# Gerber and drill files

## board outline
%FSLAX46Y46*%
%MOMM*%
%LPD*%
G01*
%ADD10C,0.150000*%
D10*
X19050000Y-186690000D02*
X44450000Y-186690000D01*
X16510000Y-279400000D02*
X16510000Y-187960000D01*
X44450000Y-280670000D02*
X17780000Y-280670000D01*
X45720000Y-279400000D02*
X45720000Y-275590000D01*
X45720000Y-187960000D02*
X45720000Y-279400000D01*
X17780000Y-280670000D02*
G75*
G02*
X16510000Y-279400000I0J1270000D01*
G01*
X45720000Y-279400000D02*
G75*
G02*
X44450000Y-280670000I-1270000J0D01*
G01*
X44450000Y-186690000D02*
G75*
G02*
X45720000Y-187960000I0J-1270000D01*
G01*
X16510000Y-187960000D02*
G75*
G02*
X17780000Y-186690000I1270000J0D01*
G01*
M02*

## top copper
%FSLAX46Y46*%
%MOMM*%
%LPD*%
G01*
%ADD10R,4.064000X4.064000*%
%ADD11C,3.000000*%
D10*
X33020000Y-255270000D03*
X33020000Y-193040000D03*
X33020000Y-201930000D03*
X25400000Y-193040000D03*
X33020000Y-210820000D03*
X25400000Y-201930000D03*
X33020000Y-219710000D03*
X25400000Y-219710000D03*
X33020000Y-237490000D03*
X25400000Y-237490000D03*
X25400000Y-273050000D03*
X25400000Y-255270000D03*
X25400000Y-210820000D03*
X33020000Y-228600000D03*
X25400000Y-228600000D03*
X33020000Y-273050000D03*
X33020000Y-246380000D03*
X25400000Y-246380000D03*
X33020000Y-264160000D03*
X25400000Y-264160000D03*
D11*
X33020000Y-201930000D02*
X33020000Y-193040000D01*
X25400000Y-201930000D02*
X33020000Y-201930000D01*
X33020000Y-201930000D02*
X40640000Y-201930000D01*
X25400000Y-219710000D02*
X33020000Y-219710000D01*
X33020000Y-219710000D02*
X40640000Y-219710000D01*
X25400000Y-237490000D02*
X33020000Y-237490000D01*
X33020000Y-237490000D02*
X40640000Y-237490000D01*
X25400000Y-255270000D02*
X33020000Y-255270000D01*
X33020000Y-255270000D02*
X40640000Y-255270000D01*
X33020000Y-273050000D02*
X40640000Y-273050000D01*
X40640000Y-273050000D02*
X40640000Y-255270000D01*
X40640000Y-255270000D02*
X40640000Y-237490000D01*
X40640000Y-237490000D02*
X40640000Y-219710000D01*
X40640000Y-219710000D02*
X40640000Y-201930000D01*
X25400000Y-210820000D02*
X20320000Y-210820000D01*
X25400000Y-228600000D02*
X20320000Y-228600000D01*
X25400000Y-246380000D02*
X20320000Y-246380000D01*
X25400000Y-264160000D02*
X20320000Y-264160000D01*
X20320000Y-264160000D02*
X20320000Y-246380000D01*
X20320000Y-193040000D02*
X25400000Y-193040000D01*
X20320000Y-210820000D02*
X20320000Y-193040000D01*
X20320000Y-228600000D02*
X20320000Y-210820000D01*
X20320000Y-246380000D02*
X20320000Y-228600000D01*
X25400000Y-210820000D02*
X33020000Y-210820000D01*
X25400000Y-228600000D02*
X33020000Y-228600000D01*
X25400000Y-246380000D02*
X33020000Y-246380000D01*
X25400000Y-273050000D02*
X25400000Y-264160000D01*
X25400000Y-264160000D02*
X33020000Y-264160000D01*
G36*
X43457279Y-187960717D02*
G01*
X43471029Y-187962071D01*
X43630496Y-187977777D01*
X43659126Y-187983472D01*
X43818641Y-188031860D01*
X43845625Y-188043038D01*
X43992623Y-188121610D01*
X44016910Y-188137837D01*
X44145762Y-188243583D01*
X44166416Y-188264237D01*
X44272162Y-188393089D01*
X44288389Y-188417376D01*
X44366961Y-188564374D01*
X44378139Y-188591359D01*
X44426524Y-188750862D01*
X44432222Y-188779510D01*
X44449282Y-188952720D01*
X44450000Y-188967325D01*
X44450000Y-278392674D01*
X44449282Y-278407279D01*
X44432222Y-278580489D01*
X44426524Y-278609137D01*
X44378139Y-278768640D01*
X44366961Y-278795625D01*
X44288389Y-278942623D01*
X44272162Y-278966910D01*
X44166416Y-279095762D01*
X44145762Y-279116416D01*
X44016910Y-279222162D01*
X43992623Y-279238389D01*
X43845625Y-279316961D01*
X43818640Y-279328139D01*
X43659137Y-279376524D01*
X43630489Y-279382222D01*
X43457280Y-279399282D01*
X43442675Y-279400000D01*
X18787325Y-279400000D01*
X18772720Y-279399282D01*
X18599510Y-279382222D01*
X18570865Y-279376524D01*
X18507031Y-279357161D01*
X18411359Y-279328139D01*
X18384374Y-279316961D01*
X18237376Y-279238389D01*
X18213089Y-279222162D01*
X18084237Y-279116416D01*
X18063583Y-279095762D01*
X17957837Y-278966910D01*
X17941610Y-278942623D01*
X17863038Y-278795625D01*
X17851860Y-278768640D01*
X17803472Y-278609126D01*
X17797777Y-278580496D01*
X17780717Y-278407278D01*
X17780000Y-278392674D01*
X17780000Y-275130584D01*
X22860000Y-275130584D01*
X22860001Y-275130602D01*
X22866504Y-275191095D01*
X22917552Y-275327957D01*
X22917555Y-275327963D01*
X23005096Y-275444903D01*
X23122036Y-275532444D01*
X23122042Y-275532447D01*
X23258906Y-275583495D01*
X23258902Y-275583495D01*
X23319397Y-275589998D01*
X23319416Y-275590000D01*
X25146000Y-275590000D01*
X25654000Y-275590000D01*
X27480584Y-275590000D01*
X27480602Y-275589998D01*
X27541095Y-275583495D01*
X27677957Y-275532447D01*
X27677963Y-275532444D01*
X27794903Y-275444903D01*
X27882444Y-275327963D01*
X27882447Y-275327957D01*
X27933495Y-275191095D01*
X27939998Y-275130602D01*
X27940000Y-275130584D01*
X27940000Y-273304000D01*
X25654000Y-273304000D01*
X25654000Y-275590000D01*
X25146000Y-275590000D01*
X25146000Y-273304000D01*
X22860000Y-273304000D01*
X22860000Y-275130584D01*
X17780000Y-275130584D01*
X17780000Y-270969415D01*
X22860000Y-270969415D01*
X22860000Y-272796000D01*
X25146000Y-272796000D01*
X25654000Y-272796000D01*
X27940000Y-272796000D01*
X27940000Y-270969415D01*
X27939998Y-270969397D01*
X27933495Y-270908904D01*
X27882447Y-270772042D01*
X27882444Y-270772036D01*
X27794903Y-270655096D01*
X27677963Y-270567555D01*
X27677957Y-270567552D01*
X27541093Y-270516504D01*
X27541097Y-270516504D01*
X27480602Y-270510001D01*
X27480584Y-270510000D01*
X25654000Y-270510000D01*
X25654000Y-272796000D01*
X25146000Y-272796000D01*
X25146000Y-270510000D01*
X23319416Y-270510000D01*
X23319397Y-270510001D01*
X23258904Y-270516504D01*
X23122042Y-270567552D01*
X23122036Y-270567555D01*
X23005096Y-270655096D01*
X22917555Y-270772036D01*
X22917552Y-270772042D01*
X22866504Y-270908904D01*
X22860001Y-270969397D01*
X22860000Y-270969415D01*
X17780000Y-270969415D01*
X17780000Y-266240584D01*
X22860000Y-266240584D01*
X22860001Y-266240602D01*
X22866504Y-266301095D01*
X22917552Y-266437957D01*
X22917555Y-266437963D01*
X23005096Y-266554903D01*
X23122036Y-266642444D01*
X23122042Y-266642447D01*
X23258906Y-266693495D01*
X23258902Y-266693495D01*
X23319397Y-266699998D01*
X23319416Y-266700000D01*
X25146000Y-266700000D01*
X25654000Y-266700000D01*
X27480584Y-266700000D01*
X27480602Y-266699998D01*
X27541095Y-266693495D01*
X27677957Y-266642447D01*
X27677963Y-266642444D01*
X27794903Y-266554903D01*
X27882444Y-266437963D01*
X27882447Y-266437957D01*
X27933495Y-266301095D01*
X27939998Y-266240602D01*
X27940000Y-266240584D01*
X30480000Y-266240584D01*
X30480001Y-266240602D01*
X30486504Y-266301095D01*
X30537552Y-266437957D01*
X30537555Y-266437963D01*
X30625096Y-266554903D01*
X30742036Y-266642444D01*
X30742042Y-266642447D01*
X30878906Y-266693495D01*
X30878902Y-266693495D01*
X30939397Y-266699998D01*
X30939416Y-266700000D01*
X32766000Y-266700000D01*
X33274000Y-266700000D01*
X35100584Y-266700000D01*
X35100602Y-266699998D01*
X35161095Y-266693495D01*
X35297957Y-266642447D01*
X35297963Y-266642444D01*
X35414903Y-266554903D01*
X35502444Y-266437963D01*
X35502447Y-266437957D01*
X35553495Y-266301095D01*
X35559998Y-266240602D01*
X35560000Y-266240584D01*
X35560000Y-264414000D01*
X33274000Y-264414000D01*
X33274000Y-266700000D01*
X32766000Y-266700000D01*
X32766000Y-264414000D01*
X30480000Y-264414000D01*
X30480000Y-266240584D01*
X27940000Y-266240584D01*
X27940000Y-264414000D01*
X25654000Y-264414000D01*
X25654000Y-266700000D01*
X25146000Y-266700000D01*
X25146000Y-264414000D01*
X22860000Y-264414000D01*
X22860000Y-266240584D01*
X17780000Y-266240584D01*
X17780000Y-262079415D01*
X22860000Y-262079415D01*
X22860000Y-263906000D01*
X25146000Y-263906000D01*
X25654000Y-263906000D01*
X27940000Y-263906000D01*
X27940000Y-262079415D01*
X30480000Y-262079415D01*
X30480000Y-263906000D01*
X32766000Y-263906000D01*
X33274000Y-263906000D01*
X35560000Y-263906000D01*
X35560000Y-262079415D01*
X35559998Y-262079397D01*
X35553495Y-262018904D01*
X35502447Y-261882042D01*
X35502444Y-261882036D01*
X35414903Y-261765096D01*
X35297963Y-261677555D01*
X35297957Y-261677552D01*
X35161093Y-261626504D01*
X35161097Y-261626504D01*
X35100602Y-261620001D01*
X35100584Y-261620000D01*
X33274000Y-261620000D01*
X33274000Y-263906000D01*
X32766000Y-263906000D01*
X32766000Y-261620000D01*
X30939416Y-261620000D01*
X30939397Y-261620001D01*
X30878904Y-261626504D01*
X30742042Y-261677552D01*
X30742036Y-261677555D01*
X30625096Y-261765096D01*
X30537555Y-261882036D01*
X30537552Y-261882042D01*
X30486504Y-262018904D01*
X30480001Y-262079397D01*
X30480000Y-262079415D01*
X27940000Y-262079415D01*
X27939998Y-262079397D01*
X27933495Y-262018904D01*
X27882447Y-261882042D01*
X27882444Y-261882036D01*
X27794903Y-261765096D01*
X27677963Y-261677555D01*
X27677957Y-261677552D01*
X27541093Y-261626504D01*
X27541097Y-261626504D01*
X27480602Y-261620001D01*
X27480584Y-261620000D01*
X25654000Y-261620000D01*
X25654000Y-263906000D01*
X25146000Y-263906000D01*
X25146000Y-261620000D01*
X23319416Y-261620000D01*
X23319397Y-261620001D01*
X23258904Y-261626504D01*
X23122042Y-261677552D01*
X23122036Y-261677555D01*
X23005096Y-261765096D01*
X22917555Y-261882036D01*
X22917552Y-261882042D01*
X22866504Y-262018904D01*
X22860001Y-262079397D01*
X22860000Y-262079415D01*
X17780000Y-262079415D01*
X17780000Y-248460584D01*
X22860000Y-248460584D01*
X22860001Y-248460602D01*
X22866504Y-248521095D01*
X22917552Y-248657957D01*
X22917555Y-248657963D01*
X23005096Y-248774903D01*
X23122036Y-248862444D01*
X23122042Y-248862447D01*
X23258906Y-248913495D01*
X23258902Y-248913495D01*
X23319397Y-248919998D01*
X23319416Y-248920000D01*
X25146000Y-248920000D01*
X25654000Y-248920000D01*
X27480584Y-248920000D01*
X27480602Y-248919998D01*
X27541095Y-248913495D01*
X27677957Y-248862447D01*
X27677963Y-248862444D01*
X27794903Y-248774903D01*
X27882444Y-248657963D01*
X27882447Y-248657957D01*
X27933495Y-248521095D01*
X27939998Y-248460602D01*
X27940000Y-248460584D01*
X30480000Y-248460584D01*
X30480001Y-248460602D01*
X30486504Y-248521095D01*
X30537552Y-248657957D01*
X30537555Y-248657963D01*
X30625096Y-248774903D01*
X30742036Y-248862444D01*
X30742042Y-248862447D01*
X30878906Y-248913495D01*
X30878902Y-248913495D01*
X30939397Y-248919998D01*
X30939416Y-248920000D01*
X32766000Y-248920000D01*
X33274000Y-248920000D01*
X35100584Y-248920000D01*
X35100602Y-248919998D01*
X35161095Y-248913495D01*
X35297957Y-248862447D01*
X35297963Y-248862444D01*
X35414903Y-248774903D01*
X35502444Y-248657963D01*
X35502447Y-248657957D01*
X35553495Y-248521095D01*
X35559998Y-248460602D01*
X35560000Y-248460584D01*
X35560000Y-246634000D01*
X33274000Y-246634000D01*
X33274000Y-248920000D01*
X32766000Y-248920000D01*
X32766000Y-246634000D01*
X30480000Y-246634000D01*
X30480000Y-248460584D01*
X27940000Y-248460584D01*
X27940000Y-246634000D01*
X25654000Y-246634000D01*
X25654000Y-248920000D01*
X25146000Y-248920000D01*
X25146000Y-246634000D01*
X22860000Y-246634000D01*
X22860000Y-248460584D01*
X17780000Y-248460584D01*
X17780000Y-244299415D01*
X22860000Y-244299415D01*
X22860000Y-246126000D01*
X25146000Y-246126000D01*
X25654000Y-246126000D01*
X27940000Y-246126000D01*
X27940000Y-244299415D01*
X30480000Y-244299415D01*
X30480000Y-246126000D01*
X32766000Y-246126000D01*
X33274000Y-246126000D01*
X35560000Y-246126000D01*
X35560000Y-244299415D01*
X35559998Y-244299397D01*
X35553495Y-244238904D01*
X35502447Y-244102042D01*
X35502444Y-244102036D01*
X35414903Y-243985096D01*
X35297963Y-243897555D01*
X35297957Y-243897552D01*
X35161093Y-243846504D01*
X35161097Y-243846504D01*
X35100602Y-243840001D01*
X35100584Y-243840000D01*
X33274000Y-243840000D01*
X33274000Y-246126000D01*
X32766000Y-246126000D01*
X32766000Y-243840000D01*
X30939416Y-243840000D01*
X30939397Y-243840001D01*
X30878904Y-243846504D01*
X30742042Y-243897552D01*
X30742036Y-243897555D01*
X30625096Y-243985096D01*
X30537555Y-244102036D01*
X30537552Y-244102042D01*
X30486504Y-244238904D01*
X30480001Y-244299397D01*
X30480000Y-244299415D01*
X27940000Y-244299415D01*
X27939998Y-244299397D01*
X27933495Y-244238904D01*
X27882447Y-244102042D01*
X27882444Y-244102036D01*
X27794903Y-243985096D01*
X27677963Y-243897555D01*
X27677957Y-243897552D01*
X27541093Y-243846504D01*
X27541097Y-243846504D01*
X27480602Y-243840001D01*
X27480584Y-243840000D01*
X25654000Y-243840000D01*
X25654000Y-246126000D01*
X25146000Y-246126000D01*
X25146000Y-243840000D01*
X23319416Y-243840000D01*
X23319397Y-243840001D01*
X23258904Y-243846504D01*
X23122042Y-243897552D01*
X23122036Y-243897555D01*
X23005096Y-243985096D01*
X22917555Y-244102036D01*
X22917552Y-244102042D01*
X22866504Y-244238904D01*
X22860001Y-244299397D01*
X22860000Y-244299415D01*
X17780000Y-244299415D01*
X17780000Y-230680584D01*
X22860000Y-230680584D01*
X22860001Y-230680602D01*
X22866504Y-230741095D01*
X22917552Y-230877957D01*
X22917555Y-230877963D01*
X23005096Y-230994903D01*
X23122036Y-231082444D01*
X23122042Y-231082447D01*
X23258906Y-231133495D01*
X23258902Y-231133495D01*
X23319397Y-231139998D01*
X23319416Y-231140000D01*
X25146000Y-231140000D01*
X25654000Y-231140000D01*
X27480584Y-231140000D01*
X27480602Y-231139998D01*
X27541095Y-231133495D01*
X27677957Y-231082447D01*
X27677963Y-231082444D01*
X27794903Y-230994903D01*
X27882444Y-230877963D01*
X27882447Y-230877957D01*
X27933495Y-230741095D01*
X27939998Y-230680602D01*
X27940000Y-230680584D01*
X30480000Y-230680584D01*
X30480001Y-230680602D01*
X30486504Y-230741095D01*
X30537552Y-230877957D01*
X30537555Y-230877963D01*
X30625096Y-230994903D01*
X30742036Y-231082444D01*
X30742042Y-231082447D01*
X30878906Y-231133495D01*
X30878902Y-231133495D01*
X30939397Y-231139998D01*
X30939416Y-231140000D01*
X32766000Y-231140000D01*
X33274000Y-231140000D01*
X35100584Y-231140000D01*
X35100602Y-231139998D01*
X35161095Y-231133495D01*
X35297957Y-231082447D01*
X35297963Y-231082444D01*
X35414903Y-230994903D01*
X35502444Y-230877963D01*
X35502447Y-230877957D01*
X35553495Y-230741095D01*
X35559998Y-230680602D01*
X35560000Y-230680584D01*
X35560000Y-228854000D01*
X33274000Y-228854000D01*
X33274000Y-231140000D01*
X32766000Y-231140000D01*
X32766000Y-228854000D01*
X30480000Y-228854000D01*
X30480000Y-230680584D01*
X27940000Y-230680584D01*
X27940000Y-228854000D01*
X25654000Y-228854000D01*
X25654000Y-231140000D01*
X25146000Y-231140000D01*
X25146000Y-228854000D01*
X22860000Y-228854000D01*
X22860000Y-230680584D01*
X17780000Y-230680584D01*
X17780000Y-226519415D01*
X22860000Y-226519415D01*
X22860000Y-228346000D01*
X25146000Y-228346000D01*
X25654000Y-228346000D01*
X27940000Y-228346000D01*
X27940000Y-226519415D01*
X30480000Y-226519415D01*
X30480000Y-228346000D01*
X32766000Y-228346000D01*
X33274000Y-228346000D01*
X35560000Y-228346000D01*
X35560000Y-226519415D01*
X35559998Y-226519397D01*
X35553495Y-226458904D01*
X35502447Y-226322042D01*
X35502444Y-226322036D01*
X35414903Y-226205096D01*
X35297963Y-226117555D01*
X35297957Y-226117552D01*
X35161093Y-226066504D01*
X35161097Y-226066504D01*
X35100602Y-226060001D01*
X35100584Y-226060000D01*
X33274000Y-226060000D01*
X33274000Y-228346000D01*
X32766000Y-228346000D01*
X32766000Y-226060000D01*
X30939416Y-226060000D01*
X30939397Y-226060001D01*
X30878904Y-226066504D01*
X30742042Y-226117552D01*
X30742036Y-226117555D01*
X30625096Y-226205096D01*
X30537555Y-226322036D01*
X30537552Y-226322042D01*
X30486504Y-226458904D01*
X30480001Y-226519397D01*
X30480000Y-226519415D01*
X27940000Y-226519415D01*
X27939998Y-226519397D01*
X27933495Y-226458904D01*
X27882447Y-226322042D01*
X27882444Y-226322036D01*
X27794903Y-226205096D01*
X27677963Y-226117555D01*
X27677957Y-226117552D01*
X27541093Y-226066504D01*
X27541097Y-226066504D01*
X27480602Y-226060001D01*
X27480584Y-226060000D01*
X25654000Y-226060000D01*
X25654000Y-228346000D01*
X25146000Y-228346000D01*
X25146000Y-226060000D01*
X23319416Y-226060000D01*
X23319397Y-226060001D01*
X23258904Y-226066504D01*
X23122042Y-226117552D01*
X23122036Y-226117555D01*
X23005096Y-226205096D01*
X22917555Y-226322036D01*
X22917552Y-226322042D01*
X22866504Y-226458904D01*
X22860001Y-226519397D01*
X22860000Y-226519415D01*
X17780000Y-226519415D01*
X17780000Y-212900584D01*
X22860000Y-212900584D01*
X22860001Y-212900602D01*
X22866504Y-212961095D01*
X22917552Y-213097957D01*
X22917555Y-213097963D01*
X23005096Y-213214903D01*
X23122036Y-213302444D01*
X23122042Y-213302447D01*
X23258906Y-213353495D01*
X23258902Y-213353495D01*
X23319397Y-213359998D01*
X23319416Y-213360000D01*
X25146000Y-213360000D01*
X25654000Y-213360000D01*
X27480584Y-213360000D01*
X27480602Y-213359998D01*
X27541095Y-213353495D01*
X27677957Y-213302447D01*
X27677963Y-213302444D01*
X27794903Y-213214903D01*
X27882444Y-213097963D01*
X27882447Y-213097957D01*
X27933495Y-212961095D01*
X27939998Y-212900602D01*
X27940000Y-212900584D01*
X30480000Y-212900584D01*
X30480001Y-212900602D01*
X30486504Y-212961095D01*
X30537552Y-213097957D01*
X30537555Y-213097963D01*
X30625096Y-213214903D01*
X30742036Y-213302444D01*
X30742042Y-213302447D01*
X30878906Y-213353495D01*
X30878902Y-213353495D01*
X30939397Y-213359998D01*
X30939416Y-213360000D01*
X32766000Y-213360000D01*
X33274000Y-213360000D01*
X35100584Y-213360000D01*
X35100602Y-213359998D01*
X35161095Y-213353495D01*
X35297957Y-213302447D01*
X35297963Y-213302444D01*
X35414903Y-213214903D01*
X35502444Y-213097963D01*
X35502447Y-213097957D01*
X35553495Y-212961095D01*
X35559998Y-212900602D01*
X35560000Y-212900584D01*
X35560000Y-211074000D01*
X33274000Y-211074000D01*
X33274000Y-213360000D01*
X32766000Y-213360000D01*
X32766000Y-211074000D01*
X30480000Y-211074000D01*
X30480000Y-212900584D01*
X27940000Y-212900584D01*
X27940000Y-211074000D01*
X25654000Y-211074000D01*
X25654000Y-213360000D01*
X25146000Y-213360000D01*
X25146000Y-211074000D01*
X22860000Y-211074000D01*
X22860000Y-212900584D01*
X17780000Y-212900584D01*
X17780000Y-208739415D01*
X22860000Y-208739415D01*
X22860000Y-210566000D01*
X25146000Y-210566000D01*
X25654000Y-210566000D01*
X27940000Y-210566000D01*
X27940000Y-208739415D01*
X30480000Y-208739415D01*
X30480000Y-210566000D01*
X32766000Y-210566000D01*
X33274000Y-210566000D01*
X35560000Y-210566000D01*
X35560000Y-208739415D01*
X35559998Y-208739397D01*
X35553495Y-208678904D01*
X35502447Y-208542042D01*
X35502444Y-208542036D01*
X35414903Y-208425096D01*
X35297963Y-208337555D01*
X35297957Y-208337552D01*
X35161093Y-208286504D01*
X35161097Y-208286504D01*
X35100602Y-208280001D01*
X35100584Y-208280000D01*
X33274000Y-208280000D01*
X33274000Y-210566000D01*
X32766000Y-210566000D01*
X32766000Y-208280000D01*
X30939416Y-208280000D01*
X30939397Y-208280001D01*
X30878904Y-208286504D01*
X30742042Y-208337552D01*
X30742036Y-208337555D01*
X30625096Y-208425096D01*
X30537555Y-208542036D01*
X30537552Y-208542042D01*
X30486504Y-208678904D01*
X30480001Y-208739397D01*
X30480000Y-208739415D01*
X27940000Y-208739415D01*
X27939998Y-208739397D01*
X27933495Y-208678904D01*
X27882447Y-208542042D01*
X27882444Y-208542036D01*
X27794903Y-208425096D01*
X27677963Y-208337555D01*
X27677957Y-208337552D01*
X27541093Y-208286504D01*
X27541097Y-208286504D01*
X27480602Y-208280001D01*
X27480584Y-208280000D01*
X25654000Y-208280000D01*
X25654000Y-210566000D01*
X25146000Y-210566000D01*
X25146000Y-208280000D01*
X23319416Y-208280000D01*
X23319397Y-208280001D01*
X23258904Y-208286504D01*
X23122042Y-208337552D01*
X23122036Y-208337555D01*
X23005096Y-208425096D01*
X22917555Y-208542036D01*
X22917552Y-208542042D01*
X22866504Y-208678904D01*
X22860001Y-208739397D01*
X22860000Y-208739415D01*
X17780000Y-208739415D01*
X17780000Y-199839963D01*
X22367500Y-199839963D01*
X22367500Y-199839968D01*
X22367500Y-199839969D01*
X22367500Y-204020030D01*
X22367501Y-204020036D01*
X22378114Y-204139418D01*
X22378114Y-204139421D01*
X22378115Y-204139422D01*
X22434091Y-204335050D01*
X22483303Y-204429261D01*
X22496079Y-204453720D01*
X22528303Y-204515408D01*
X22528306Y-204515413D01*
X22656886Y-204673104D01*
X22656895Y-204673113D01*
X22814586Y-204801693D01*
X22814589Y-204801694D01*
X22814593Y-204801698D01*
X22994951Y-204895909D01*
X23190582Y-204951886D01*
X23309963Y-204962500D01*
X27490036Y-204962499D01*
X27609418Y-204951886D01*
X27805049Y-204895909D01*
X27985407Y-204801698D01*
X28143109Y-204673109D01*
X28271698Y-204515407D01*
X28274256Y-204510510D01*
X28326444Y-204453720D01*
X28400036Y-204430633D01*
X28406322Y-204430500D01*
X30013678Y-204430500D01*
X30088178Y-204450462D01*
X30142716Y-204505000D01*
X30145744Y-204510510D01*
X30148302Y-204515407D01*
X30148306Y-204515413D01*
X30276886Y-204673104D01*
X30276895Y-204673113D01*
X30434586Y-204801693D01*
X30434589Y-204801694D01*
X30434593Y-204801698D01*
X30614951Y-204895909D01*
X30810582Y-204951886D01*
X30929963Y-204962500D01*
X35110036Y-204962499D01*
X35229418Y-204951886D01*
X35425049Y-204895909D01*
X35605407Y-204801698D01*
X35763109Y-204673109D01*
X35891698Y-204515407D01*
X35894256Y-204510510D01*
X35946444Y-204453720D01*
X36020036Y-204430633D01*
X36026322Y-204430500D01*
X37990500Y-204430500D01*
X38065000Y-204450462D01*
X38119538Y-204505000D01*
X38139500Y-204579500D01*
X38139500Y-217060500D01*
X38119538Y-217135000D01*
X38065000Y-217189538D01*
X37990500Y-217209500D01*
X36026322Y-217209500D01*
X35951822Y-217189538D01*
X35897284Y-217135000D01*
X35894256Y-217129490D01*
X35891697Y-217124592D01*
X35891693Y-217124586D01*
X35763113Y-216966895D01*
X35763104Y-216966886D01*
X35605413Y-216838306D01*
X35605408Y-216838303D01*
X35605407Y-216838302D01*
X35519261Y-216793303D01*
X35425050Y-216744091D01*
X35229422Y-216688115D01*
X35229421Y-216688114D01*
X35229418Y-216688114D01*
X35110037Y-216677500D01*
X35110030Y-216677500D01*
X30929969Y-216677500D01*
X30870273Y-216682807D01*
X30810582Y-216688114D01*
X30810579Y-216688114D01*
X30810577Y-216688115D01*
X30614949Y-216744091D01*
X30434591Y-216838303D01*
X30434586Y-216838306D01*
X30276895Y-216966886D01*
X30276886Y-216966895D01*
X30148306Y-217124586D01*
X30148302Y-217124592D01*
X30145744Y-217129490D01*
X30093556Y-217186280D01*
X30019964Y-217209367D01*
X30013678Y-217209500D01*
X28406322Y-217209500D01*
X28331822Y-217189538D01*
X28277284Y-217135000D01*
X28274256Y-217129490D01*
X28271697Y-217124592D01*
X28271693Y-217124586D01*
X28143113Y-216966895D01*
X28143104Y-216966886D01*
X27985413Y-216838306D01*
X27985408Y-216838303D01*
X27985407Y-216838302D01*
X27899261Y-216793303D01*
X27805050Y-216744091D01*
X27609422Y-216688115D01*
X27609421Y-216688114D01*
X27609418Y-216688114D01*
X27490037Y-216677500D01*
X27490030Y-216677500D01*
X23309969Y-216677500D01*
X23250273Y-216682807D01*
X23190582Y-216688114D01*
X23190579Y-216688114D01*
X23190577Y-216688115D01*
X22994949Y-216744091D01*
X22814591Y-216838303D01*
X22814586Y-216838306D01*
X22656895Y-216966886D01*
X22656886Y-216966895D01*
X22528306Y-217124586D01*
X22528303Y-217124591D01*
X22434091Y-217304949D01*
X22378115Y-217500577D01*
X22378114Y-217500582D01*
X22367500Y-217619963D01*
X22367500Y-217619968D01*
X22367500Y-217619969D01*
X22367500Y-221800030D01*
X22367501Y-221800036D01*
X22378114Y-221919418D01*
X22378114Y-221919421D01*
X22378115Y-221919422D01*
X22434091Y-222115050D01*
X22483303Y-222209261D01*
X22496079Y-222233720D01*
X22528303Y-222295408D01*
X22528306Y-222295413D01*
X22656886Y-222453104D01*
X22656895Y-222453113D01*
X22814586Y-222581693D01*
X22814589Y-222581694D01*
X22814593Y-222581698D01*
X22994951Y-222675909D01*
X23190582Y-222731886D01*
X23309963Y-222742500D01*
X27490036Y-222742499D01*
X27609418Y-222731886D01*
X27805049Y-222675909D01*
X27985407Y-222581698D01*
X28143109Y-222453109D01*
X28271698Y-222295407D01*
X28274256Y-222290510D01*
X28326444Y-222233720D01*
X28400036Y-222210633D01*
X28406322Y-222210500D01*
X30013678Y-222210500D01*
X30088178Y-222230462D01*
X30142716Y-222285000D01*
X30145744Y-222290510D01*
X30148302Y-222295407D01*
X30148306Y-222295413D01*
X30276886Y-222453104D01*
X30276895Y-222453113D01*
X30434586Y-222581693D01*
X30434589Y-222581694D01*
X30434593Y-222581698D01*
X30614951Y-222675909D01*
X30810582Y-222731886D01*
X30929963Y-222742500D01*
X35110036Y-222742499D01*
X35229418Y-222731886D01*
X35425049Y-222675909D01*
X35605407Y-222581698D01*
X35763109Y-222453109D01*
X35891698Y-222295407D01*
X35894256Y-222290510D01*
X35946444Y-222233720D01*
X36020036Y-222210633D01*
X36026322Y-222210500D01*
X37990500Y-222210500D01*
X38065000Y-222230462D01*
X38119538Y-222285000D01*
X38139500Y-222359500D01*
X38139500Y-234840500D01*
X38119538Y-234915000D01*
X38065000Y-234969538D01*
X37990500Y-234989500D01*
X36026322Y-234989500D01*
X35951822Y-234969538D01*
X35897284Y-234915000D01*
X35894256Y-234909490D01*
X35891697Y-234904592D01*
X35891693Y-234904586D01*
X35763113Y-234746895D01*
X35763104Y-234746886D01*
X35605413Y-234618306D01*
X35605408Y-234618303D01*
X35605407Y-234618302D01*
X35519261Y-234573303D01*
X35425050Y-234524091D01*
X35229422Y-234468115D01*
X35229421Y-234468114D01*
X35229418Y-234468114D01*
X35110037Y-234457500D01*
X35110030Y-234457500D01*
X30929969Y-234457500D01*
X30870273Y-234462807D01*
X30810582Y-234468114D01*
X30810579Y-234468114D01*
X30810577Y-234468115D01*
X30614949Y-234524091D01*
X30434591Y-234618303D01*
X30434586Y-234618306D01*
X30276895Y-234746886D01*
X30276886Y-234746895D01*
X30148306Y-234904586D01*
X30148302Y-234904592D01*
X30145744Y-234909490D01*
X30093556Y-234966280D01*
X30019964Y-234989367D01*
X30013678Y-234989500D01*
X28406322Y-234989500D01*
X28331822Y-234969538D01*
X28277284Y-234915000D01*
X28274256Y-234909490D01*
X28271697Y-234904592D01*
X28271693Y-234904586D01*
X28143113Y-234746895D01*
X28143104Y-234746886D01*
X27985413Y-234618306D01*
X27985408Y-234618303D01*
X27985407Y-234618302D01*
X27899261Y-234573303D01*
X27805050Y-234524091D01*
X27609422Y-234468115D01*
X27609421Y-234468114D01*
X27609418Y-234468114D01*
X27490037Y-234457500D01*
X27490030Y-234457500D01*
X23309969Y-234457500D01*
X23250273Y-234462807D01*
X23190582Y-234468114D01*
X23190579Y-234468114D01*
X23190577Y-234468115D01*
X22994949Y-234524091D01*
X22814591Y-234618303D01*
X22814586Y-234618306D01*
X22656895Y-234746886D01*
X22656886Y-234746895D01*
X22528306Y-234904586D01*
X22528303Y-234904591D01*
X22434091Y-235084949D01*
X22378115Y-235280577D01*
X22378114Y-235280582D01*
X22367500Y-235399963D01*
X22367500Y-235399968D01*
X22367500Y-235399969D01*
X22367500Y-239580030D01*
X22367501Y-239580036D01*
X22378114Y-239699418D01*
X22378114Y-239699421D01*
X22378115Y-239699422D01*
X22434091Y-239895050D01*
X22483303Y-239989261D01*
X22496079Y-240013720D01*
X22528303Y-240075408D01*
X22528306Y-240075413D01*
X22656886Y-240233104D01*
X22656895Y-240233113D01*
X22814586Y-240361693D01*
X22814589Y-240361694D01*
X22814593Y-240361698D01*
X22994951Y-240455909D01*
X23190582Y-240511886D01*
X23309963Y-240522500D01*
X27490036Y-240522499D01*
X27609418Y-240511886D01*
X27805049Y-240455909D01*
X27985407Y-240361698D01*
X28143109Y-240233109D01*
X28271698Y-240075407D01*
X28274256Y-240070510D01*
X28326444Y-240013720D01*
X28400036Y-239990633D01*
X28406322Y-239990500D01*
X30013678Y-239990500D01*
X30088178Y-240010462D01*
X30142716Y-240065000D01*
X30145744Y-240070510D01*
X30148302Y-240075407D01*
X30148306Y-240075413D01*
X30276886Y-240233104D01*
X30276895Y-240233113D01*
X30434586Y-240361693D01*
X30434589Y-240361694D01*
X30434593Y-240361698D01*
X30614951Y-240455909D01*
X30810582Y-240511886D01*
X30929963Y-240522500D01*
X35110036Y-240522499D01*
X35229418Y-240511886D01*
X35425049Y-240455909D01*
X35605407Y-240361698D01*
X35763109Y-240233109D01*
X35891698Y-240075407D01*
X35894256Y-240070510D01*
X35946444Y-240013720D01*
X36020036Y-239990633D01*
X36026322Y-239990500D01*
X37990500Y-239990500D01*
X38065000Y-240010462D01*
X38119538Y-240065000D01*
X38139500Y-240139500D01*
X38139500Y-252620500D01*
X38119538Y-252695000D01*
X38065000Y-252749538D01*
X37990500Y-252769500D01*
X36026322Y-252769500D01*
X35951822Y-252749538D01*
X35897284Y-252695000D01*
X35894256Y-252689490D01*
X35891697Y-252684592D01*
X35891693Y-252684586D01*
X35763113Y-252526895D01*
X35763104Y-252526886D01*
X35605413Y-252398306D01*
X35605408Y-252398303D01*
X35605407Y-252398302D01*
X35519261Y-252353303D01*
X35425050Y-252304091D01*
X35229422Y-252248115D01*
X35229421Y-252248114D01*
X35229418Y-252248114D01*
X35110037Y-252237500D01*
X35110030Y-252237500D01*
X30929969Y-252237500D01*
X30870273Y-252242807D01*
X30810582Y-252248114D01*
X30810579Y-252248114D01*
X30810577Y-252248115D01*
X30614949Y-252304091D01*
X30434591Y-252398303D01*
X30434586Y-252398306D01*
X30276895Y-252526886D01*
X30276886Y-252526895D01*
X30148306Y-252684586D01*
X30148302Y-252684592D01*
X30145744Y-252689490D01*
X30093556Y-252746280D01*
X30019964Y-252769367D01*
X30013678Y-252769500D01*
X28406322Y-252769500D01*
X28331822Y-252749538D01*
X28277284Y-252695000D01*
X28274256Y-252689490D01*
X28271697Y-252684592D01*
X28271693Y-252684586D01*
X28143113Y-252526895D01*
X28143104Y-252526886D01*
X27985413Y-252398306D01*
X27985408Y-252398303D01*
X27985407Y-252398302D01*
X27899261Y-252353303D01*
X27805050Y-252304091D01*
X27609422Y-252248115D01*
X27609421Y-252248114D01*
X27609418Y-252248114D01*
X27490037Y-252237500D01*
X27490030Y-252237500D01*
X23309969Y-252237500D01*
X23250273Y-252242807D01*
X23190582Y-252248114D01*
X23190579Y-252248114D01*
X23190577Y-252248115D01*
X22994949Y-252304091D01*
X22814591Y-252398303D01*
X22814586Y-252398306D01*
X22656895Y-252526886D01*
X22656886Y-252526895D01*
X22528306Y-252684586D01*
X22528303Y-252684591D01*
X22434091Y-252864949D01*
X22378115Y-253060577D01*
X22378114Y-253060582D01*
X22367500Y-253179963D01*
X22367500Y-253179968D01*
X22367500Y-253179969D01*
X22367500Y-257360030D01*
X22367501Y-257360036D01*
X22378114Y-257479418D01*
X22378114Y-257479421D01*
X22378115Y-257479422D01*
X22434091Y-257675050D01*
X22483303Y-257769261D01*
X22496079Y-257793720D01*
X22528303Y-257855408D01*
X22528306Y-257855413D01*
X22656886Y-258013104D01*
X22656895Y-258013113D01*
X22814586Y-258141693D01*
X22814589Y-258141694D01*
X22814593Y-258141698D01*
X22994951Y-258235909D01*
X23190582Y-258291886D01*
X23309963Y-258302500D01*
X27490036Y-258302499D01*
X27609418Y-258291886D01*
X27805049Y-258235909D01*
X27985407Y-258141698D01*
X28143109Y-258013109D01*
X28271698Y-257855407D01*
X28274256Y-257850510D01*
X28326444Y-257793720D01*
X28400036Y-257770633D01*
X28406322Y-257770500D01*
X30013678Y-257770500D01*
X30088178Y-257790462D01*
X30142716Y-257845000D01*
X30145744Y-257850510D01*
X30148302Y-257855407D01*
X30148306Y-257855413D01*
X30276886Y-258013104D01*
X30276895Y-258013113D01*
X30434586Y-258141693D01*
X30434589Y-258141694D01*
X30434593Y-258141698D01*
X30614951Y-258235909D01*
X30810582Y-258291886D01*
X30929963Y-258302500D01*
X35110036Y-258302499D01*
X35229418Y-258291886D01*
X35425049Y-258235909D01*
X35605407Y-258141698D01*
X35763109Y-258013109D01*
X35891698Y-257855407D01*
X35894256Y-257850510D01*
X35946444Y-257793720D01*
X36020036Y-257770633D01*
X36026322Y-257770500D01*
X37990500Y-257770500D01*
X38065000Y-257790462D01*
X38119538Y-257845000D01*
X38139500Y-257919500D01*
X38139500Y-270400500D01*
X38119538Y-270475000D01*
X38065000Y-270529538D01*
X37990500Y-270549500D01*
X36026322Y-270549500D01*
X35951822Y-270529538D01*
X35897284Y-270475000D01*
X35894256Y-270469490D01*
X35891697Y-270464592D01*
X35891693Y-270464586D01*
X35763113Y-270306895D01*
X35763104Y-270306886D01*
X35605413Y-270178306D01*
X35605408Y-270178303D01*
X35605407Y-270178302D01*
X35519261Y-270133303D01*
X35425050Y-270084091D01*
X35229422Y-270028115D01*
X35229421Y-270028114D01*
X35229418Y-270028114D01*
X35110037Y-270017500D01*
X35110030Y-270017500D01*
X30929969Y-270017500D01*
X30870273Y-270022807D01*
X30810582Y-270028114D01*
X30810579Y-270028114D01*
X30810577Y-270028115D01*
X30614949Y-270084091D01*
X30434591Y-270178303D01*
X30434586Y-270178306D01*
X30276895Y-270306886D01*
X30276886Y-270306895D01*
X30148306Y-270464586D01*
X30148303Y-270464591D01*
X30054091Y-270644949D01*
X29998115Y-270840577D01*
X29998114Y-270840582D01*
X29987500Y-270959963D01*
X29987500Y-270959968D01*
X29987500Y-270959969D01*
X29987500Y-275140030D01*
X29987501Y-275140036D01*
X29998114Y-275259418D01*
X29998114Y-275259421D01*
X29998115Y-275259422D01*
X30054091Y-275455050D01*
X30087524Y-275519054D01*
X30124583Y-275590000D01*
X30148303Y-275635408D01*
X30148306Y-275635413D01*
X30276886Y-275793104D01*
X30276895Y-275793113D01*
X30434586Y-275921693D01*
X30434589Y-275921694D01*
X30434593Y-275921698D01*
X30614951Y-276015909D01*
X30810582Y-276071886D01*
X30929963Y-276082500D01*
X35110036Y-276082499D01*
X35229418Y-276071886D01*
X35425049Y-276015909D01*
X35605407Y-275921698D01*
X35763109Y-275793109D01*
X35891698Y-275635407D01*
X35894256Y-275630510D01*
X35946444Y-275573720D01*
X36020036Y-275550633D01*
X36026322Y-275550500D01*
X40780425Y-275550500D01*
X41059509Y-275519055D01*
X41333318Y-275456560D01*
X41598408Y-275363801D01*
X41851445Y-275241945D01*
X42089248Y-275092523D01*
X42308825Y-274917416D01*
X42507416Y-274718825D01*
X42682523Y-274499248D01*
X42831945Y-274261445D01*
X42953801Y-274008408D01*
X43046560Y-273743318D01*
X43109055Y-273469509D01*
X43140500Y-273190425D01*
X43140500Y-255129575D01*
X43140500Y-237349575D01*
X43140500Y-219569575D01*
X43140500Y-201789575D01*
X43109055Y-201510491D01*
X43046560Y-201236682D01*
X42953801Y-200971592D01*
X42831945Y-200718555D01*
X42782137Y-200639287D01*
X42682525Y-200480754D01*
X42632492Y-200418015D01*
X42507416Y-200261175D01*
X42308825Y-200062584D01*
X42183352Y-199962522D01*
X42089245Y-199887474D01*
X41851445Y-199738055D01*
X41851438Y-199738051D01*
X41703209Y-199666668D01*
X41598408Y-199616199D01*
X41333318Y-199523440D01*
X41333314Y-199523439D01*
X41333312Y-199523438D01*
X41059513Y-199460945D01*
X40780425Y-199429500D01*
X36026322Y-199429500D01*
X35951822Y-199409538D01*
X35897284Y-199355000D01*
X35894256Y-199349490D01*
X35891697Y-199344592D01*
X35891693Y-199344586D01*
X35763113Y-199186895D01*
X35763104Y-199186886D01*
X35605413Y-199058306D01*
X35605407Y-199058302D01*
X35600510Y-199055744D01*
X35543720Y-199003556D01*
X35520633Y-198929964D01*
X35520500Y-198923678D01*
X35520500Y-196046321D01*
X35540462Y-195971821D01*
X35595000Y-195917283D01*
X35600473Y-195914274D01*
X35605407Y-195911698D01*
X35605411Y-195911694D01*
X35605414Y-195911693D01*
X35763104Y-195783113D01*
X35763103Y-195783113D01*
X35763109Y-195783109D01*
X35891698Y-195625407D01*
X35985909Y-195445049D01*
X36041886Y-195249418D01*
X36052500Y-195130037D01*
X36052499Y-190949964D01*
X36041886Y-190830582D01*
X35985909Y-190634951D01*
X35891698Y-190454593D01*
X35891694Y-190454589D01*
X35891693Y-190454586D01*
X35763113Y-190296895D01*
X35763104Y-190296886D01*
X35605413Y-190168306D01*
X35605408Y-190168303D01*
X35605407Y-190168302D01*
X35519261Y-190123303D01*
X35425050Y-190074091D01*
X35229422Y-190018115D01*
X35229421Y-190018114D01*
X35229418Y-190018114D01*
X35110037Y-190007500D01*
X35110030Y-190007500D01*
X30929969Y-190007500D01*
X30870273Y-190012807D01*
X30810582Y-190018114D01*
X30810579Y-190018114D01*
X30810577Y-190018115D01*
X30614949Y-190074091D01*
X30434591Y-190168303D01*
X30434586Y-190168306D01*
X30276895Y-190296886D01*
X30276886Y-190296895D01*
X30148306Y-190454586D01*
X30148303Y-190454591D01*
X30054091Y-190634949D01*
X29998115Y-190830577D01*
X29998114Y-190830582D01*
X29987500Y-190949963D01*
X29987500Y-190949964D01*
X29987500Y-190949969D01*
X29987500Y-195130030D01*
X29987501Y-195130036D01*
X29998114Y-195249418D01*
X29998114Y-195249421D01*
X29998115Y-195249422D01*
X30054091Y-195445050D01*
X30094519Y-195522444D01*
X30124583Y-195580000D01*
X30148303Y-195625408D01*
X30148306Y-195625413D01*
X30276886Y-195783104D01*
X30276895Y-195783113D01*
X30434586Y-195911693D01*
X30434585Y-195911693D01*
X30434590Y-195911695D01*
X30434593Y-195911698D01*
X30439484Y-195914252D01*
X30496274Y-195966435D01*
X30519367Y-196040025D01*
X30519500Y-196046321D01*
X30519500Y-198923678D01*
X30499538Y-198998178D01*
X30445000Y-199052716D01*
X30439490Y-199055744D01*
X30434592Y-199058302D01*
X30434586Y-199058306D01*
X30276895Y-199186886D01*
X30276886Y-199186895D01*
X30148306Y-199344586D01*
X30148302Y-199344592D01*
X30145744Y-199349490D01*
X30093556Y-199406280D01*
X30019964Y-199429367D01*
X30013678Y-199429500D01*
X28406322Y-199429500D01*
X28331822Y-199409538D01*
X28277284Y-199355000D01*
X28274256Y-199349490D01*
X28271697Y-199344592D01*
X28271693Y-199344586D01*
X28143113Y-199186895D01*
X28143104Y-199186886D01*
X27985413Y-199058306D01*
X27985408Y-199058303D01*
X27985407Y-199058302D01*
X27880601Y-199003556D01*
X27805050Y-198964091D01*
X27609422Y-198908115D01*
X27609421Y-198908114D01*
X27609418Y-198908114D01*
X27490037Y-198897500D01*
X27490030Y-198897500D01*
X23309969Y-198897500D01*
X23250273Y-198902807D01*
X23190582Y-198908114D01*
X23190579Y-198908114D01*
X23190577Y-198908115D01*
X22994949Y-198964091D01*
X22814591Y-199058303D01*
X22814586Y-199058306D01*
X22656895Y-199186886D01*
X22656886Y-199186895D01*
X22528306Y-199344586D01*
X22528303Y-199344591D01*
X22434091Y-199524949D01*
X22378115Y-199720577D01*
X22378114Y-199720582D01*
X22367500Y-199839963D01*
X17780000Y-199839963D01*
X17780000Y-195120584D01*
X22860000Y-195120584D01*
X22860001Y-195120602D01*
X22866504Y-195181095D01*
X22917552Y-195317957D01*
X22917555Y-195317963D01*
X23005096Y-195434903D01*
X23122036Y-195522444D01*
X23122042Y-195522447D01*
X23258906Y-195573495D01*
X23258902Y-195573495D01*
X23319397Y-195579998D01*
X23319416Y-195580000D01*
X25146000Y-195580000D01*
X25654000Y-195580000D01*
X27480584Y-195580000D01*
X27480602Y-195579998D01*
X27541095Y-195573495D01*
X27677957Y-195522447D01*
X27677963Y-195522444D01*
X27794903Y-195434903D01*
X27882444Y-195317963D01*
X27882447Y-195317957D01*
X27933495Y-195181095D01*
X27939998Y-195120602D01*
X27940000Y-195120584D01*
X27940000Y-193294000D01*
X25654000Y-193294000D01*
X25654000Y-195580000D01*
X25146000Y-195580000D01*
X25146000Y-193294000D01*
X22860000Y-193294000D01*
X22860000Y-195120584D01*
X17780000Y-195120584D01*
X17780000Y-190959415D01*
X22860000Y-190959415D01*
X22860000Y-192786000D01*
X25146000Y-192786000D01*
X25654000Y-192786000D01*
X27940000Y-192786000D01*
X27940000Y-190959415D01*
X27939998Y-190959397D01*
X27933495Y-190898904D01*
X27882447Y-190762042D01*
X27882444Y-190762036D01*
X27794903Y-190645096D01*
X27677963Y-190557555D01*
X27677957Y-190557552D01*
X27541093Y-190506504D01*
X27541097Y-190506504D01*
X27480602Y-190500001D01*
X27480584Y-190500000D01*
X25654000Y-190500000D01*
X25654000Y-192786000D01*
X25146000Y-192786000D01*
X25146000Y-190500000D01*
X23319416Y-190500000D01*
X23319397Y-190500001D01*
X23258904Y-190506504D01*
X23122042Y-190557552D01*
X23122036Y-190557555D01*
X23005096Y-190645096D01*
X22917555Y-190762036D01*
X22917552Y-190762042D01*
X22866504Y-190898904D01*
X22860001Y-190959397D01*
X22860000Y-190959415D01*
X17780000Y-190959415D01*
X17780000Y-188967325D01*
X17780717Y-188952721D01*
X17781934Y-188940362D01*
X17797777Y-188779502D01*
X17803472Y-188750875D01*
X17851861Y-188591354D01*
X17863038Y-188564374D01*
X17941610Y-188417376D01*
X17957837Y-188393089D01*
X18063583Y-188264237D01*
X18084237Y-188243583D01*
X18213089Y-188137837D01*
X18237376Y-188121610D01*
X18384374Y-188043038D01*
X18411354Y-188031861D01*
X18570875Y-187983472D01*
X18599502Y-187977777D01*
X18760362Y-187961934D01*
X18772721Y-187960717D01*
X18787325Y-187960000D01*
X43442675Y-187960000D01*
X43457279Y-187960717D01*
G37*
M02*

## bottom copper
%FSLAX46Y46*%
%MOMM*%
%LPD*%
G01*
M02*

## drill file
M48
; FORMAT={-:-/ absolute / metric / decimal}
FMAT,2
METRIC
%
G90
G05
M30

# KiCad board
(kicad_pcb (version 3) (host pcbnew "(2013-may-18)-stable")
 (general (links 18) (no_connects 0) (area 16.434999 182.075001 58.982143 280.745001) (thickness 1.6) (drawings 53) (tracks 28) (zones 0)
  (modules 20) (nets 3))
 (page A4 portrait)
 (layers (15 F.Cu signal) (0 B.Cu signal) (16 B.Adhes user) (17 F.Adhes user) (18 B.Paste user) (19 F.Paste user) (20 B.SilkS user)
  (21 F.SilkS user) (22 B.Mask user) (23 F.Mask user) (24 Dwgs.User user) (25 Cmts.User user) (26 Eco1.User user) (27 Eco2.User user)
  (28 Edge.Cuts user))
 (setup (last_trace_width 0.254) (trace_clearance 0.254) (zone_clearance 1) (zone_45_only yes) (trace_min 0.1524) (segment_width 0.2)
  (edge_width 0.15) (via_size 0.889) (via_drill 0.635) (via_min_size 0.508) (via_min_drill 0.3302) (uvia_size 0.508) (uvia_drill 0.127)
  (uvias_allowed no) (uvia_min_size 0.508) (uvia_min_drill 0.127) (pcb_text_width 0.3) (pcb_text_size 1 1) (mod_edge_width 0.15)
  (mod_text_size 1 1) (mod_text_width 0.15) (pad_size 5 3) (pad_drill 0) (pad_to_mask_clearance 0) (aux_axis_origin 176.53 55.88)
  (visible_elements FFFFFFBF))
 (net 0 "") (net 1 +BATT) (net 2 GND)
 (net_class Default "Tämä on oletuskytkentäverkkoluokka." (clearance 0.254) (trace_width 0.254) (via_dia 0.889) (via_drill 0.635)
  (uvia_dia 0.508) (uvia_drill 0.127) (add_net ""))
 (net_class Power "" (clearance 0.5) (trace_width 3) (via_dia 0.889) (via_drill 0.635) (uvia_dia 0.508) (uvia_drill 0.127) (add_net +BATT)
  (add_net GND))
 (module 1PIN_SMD (layer F.Cu) (at 33.02 255.27)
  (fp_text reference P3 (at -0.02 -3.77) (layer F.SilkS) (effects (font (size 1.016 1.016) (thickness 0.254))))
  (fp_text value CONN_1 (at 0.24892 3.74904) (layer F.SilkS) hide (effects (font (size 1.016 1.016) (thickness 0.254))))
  (pad 1 smd rect (at 0 0) (size 4.064 4.064) (layers F.Cu F.Paste F.SilkS F.Mask) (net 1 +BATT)))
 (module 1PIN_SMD (layer F.Cu) (at 33.02 193.04)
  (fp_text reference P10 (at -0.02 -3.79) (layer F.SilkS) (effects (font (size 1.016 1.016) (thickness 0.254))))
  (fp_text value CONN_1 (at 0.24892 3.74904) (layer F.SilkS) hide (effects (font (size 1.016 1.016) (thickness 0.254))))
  (pad 1 smd rect (at 0 0) (size 4.064 4.064) (layers F.Cu F.Paste F.SilkS F.Mask) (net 1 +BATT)))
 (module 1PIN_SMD (layer F.Cu) (at 33.02 201.93)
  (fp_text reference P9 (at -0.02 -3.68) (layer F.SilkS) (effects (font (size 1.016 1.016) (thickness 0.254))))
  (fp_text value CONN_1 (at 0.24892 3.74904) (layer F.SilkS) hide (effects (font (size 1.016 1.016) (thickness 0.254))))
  (pad 1 smd rect (at 0 0) (size 4.064 4.064) (layers F.Cu F.Paste F.SilkS F.Mask) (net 1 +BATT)))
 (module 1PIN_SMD (layer F.Cu) (at 25.4 193.04)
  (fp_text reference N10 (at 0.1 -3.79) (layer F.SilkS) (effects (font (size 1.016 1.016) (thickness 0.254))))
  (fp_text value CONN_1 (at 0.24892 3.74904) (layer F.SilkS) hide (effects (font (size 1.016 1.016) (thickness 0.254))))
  (pad 1 smd rect (at 0 0) (size 4.064 4.064) (layers F.Cu F.Paste F.SilkS F.Mask) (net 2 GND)))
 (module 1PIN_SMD (layer F.Cu) (at 33.02 210.82)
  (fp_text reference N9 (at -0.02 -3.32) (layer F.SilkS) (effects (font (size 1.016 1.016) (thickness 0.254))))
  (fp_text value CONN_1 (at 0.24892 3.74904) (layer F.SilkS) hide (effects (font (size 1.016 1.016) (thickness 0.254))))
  (pad 1 smd rect (at 0 0) (size 4.064 4.064) (layers F.Cu F.Paste F.SilkS F.Mask) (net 2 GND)))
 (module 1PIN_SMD (layer F.Cu) (at 25.4 201.93)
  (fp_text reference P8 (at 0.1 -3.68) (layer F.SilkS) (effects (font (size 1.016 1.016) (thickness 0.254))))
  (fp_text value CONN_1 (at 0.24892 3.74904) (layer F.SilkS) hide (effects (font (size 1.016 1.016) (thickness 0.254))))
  (pad 1 smd rect (at 0 0) (size 4.064 4.064) (layers F.Cu F.Paste F.SilkS F.Mask) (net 1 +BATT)))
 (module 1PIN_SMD (layer F.Cu) (at 33.02 219.71)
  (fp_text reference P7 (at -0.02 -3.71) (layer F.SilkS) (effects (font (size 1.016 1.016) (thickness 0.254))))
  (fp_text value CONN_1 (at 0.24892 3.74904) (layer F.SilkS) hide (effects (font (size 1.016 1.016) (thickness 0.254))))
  (pad 1 smd rect (at 0 0) (size 4.064 4.064) (layers F.Cu F.Paste F.SilkS F.Mask) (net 1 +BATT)))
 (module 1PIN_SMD (layer F.Cu) (at 25.4 219.71)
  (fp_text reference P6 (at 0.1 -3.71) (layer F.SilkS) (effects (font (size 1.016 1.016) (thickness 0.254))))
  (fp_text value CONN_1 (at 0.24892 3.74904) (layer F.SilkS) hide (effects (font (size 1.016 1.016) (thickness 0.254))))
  (pad 1 smd rect (at 0 0) (size 4.064 4.064) (layers F.Cu F.Paste F.SilkS F.Mask) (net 1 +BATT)))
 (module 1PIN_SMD (layer F.Cu) (at 33.02 237.49)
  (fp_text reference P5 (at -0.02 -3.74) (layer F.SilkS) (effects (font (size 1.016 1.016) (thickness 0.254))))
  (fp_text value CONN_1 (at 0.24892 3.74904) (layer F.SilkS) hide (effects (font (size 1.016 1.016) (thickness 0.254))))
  (pad 1 smd rect (at 0 0) (size 4.064 4.064) (layers F.Cu F.Paste F.SilkS F.Mask) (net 1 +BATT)))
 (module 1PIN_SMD (layer F.Cu) (at 25.4 237.49)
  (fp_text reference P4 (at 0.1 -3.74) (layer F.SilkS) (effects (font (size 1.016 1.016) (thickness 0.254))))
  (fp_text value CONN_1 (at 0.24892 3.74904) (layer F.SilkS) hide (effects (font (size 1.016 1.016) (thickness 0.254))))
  (pad 1 smd rect (at 0 0) (size 4.064 4.064) (layers F.Cu F.Paste F.SilkS F.Mask) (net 1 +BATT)))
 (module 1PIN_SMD (layer F.Cu) (at 25.4 273.05)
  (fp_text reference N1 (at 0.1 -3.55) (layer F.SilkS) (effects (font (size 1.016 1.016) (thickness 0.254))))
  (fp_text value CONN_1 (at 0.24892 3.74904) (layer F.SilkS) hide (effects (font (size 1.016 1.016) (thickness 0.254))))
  (pad 1 smd rect (at 0 0) (size 4.064 4.064) (layers F.Cu F.Paste F.SilkS F.Mask) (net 2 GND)))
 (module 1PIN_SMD (layer F.Cu) (at 25.4 255.27)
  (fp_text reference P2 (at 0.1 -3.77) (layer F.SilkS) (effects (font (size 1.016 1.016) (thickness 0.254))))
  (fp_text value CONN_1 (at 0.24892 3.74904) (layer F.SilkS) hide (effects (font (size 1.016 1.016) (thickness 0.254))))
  (pad 1 smd rect (at 0 0) (size 4.064 4.064) (layers F.Cu F.Paste F.SilkS F.Mask) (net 1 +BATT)))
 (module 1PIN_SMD (layer F.Cu) (at 25.4 210.82)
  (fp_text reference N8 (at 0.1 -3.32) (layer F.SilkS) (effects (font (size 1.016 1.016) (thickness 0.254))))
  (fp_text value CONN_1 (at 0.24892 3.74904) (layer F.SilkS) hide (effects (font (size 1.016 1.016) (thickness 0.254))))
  (pad 1 smd rect (at 0 0) (size 4.064 4.064) (layers F.Cu F.Paste F.SilkS F.Mask) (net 2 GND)))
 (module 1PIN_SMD (layer F.Cu) (at 33.02 228.6)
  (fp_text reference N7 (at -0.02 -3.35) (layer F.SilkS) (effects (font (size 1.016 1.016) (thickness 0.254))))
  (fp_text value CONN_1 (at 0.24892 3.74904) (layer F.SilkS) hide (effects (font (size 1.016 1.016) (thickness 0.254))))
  (pad 1 smd rect (at 0 0) (size 4.064 4.064) (layers F.Cu F.Paste F.SilkS F.Mask) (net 2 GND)))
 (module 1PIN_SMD (layer F.Cu) (at 25.4 228.6)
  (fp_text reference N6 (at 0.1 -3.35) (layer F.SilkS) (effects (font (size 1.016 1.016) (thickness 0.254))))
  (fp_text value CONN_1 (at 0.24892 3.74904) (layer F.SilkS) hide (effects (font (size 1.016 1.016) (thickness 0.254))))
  (pad 1 smd rect (at 0 0) (size 4.064 4.064) (layers F.Cu F.Paste F.SilkS F.Mask) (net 2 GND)))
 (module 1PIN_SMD (layer F.Cu) (at 33.02 273.05)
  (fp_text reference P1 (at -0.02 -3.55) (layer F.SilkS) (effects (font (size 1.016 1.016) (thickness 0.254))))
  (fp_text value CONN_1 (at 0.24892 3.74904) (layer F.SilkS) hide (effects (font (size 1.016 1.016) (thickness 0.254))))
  (pad 1 smd rect (at 0 0) (size 4.064 4.064) (layers F.Cu F.Paste F.SilkS F.Mask) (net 1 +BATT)))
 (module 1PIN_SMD (layer F.Cu) (at 33.02 246.38)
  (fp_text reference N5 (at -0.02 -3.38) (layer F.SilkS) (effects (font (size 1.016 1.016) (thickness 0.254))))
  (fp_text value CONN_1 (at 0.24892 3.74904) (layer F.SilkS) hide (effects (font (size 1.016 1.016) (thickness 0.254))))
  (pad 1 smd rect (at 0 0) (size 4.064 4.064) (layers F.Cu F.Paste F.SilkS F.Mask) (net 2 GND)))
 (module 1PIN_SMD (layer F.Cu) (at 25.4 246.38)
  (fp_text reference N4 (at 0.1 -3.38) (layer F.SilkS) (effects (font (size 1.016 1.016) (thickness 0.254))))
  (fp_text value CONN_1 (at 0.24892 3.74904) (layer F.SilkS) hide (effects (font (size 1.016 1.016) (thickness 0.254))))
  (pad 1 smd rect (at 0 0) (size 4.064 4.064) (layers F.Cu F.Paste F.SilkS F.Mask) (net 2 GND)))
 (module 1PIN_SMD (layer F.Cu) (at 33.02 264.16)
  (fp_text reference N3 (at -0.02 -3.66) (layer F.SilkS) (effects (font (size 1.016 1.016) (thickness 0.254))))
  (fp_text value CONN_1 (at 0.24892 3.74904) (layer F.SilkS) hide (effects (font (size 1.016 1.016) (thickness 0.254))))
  (pad 1 smd rect (at 0 0) (size 4.064 4.064) (layers F.Cu F.Paste F.SilkS F.Mask) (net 2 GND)))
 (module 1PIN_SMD (layer F.Cu) (at 25.4 264.16)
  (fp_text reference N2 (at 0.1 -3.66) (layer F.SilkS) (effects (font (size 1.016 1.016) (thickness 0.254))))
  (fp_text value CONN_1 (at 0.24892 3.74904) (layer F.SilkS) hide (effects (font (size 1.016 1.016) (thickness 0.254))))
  (pad 1 smd rect (at 0 0) (size 4.064 4.064) (layers F.Cu F.Paste F.SilkS F.Mask) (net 2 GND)))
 (gr_line (start 19.05 186.69) (end 44.45 186.69) (angle 90) (layer Edge.Cuts) (width 0.15))
 (gr_line (start 16.51 279.4) (end 16.51 187.96) (angle 90) (layer Edge.Cuts) (width 0.15))
 (gr_line (start 44.45 280.67) (end 17.78 280.67) (angle 90) (layer Edge.Cuts) (width 0.15))
 (gr_line (start 45.72 279.4) (end 45.72 275.59) (angle 90) (layer Edge.Cuts) (width 0.15))
 (gr_line (start 45.72 187.96) (end 45.72 279.4) (angle 90) (layer Edge.Cuts) (width 0.15))
 (gr_arc (start 17.78 279.4) (end 17.78 280.67) (angle 90) (layer Edge.Cuts) (width 0.15))
 (gr_arc (start 44.45 279.4) (end 45.72 279.4) (angle 90) (layer Edge.Cuts) (width 0.15))
 (gr_arc (start 44.45 187.96) (end 44.45 186.69) (angle 90) (layer Edge.Cuts) (width 0.15))
 (gr_arc (start 17.78 187.96) (end 16.51 187.96) (angle 90) (layer Edge.Cuts) (width 0.15))
 (segment (start 33.02 201.93) (end 33.02 193.04) (width 3) (layer F.Cu) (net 1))
 (segment (start 25.4 201.93) (end 33.02 201.93) (width 3) (layer F.Cu) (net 1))
 (segment (start 33.02 201.93) (end 40.64 201.93) (width 3) (layer F.Cu) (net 1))
 (segment (start 25.4 219.71) (end 33.02 219.71) (width 3) (layer F.Cu) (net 1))
 (segment (start 33.02 219.71) (end 40.64 219.71) (width 3) (layer F.Cu) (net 1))
 (segment (start 25.4 237.49) (end 33.02 237.49) (width 3) (layer F.Cu) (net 1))
 (segment (start 33.02 237.49) (end 40.64 237.49) (width 3) (layer F.Cu) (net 1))
 (segment (start 25.4 255.27) (end 33.02 255.27) (width 3) (layer F.Cu) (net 1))
 (segment (start 33.02 255.27) (end 40.64 255.27) (width 3) (layer F.Cu) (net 1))
 (segment (start 33.02 273.05) (end 40.64 273.05) (width 3) (layer F.Cu) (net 1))
 (segment (start 40.64 273.05) (end 40.64 255.27) (width 3) (layer F.Cu) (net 1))
 (segment (start 40.64 255.27) (end 40.64 237.49) (width 3) (layer F.Cu) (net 1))
 (segment (start 40.64 237.49) (end 40.64 219.71) (width 3) (layer F.Cu) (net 1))
 (segment (start 40.64 219.71) (end 40.64 201.93) (width 3) (layer F.Cu) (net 1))
 (segment (start 25.4 210.82) (end 20.32 210.82) (width 3) (layer F.Cu) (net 2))
 (segment (start 25.4 228.6) (end 20.32 228.6) (width 3) (layer F.Cu) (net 2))
 (segment (start 25.4 246.38) (end 20.32 246.38) (width 3) (layer F.Cu) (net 2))
 (segment (start 25.4 264.16) (end 20.32 264.16) (width 3) (layer F.Cu) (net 2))
 (segment (start 20.32 264.16) (end 20.32 246.38) (width 3) (layer F.Cu) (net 2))
 (segment (start 20.32 193.04) (end 25.4 193.04) (width 3) (layer F.Cu) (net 2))
 (segment (start 20.32 210.82) (end 20.32 193.04) (width 3) (layer F.Cu) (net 2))
 (segment (start 20.32 228.6) (end 20.32 210.82) (width 3) (layer F.Cu) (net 2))
 (segment (start 20.32 246.38) (end 20.32 228.6) (width 3) (layer F.Cu) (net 2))
 (segment (start 25.4 210.82) (end 33.02 210.82) (width 3) (layer F.Cu) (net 2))
 (segment (start 25.4 228.6) (end 33.02 228.6) (width 3) (layer F.Cu) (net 2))
 (segment (start 25.4 246.38) (end 33.02 246.38) (width 3) (layer F.Cu) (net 2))
 (segment (start 25.4 273.05) (end 25.4 264.16) (width 3) (layer F.Cu) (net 2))
 (segment (start 25.4 264.16) (end 33.02 264.16) (width 3) (layer F.Cu) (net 2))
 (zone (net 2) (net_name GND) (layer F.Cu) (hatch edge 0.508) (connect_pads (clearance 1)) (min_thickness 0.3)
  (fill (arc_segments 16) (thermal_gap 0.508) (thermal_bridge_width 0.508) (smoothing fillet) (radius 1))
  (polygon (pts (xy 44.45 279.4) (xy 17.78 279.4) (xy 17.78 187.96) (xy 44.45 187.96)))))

